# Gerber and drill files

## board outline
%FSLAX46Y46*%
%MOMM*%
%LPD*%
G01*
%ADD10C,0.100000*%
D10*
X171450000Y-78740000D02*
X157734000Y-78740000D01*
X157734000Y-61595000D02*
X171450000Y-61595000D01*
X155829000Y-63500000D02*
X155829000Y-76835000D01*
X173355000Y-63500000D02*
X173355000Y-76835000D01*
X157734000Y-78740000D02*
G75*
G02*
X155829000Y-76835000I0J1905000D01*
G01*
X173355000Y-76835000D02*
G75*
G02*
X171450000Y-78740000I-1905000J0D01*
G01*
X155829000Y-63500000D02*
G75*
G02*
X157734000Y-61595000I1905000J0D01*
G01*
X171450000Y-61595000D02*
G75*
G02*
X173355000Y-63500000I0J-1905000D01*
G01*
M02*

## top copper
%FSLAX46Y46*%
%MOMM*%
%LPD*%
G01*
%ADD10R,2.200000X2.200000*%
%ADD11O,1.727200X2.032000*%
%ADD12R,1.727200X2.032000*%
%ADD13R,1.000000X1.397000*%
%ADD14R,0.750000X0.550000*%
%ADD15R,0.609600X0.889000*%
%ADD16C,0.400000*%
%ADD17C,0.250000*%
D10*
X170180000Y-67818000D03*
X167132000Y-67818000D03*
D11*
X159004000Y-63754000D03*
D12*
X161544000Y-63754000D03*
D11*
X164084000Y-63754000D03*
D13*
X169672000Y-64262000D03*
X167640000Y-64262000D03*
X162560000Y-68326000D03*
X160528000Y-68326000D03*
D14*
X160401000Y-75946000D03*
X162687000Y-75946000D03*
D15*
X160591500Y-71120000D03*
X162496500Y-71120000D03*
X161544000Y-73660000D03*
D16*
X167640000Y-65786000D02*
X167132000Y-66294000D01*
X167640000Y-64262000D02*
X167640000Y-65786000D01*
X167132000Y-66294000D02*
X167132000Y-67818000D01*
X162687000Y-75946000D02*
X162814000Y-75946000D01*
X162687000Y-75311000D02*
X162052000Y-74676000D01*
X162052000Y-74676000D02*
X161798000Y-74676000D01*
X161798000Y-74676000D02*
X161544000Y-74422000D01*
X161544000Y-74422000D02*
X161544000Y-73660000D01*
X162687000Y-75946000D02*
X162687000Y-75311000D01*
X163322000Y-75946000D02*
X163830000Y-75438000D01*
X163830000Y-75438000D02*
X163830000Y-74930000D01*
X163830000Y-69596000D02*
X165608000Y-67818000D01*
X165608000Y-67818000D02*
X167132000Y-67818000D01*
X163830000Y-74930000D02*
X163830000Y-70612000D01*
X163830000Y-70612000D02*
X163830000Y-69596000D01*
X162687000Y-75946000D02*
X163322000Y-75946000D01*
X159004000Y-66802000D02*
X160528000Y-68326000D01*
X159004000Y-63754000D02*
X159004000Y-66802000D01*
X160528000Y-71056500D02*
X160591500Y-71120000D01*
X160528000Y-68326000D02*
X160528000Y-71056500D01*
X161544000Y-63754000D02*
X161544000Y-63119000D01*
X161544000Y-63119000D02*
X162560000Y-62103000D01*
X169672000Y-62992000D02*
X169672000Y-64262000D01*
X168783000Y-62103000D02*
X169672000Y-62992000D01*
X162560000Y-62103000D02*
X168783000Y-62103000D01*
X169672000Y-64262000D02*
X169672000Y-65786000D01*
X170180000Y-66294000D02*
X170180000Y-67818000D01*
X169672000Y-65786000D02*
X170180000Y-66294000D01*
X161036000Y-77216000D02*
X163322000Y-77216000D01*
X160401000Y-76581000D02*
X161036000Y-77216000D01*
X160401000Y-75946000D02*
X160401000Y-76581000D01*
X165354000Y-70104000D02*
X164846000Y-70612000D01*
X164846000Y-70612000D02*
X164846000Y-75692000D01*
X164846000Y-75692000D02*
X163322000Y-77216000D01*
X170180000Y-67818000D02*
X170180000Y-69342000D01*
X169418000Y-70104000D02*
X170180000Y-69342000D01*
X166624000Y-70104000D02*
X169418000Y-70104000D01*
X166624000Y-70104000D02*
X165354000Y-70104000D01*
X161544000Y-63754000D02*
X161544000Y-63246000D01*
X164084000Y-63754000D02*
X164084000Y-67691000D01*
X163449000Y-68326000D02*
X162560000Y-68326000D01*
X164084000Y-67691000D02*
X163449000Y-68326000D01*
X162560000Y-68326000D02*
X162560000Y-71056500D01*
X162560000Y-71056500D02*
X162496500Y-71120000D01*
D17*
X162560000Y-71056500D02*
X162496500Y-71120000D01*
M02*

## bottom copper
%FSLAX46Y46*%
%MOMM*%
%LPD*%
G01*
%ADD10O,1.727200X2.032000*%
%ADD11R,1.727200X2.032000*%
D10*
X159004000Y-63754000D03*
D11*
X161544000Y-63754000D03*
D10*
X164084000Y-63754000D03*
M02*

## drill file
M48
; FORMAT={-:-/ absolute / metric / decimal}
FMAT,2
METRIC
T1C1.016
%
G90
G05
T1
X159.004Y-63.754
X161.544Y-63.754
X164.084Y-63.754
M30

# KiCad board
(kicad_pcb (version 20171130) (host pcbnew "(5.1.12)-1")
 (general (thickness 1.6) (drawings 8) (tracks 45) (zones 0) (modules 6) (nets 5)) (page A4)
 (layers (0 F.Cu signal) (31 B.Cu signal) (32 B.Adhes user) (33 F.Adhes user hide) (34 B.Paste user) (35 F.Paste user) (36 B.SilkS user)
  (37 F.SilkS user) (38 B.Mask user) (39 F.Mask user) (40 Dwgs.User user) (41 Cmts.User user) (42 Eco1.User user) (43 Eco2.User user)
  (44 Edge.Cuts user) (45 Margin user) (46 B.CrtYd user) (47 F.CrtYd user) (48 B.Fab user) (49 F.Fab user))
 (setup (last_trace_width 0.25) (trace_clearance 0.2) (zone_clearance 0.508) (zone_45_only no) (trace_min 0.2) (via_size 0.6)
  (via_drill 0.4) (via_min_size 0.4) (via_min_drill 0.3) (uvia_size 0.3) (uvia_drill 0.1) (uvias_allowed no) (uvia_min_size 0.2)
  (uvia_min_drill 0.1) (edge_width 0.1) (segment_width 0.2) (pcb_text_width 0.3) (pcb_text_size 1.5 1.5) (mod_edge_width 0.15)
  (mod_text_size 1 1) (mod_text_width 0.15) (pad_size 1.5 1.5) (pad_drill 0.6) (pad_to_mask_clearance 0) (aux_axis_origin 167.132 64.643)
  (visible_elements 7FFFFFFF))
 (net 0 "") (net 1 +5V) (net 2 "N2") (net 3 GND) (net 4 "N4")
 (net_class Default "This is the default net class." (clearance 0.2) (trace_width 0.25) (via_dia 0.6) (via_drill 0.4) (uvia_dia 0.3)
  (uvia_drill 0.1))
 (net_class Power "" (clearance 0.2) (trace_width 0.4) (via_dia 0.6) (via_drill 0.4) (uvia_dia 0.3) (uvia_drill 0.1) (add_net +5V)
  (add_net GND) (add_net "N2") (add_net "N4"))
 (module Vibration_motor (layer F.Cu) (at 168.656 67.818 180)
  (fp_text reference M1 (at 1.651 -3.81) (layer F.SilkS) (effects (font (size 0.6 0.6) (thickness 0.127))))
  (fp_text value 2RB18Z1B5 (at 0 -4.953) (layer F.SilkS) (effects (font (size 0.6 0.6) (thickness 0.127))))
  (pad 1 smd rect (at -1.524 0 180) (size 2.2 2.2) (layers F.Cu F.Paste F.Mask) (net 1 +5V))
  (pad 2 smd rect (at 1.524 0 180) (size 2.2 2.2) (layers F.Cu F.Paste F.Mask) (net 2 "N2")))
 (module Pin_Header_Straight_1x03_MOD (layer F.Cu) (at 159.004 63.754 90)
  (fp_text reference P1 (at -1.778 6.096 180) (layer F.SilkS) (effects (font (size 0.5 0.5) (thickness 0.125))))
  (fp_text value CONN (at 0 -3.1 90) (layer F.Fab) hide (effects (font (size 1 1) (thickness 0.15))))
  (pad 1 thru_hole oval (at 0 0 90) (size 2.032 1.7272) (drill 1.016) (layers *.Cu *.Mask F.SilkS) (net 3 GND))
  (pad 2 thru_hole rect (at 0 2.54 90) (size 2.032 1.7272) (drill 1.016) (layers *.Cu *.Mask F.SilkS) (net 1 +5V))
  (pad 3 thru_hole oval (at 0 5.08 90) (size 2.032 1.7272) (drill 1.016) (layers *.Cu *.Mask F.SilkS) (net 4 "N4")))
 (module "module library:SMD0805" (layer F.Cu) (at 168.656 64.262 180)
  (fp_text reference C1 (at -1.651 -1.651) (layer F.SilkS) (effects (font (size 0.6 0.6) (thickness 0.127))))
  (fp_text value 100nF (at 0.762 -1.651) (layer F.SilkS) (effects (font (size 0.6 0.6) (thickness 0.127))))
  (pad 1 smd rect (at -1.016 0 180) (size 1 1.397) (layers F.Cu F.Paste F.Mask) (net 1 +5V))
  (pad 2 smd rect (at 1.016 0 180) (size 1 1.397) (layers F.Cu F.Paste F.Mask) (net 2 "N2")))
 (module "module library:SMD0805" (layer F.Cu) (at 161.544 68.326 180)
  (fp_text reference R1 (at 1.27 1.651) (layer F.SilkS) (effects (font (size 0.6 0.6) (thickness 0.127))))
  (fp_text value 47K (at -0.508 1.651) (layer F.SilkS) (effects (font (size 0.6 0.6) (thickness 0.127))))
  (pad 1 smd rect (at -1.016 0 180) (size 1 1.397) (layers F.Cu F.Paste F.Mask) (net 4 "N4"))
  (pad 2 smd rect (at 1.016 0 180) (size 1 1.397) (layers F.Cu F.Paste F.Mask) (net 3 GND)))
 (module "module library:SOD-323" (layer F.Cu) (at 161.544 75.946)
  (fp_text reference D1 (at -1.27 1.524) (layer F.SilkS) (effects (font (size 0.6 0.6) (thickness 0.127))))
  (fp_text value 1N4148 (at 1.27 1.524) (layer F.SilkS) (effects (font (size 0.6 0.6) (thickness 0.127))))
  (pad 1 smd rect (at -1.143 0) (size 0.75 0.55) (layers F.Cu F.Paste F.Mask) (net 1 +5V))
  (pad 2 smd rect (at 1.143 0) (size 0.75 0.55) (layers F.Cu F.Paste F.Mask) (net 2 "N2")))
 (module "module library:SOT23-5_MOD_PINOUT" (layer F.Cu) (at 161.544 72.39 180)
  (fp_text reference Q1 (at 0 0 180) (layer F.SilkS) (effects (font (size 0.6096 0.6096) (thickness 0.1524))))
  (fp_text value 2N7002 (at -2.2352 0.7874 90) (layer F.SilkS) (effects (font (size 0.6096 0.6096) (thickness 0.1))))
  (pad 3 smd rect (at 0.9525 1.27 180) (size 0.6096 0.889) (layers F.Cu F.Paste F.Mask) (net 3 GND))
  (pad 2 smd rect (at -0.9525 1.27 180) (size 0.6096 0.889) (layers F.Cu F.Paste F.Mask) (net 4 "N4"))
  (pad 1 smd rect (at 0 -1.27 180) (size 0.6096 0.889) (layers F.Cu F.Paste F.Mask) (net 2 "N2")))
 (gr_line (start 171.45 78.74) (end 157.734 78.74) (angle 90) (layer Edge.Cuts) (width 0.1))
 (gr_line (start 157.734 61.595) (end 171.45 61.595) (angle 90) (layer Edge.Cuts) (width 0.1))
 (gr_line (start 155.829 63.5) (end 155.829 76.835) (angle 90) (layer Edge.Cuts) (width 0.1))
 (gr_line (start 173.355 63.5) (end 173.355 76.835) (angle 90) (layer Edge.Cuts) (width 0.1))
 (gr_arc (start 157.734 76.835) (end 157.734 78.74) (angle 90) (layer Edge.Cuts) (width 0.1))
 (gr_arc (start 171.45 76.835) (end 173.355 76.835) (angle 90) (layer Edge.Cuts) (width 0.1))
 (gr_arc (start 157.734 63.5) (end 155.829 63.5) (angle 90) (layer Edge.Cuts) (width 0.1))
 (gr_arc (start 171.45 63.5) (end 171.45 61.595) (angle 90) (layer Edge.Cuts) (width 0.1))
 (segment (start 167.64 65.786) (end 167.132 66.294) (width 0.4) (layer F.Cu) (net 2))
 (segment (start 167.64 64.262) (end 167.64 65.786) (width 0.4) (layer F.Cu) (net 2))
 (segment (start 167.132 66.294) (end 167.132 67.818) (width 0.4) (layer F.Cu) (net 2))
 (segment (start 162.687 75.946) (end 162.814 75.946) (width 0.4) (layer F.Cu) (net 2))
 (segment (start 162.687 75.311) (end 162.052 74.676) (width 0.4) (layer F.Cu) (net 2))
 (segment (start 162.052 74.676) (end 161.798 74.676) (width 0.4) (layer F.Cu) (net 2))
 (segment (start 161.798 74.676) (end 161.544 74.422) (width 0.4) (layer F.Cu) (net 2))
 (segment (start 161.544 74.422) (end 161.544 73.66) (width 0.4) (layer F.Cu) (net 2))
 (segment (start 162.687 75.946) (end 162.687 75.311) (width 0.4) (layer F.Cu) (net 2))
 (segment (start 163.322 75.946) (end 163.83 75.438) (width 0.4) (layer F.Cu) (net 2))
 (segment (start 163.83 75.438) (end 163.83 74.93) (width 0.4) (layer F.Cu) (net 2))
 (segment (start 163.83 69.596) (end 165.608 67.818) (width 0.4) (layer F.Cu) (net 2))
 (segment (start 165.608 67.818) (end 167.132 67.818) (width 0.4) (layer F.Cu) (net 2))
 (segment (start 163.83 74.93) (end 163.83 70.612) (width 0.4) (layer F.Cu) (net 2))
 (segment (start 163.83 70.612) (end 163.83 69.596) (width 0.4) (layer F.Cu) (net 2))
 (segment (start 162.687 75.946) (end 163.322 75.946) (width 0.4) (layer F.Cu) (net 2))
 (segment (start 159.004 66.802) (end 160.528 68.326) (width 0.4) (layer F.Cu) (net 3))
 (segment (start 159.004 63.754) (end 159.004 66.802) (width 0.4) (layer F.Cu) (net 3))
 (segment (start 160.528 71.0565) (end 160.5915 71.12) (width 0.4) (layer F.Cu) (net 3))
 (segment (start 160.528 68.326) (end 160.528 71.0565) (width 0.4) (layer F.Cu) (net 3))
 (segment (start 161.544 63.754) (end 161.544 63.119) (width 0.4) (layer F.Cu) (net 1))
 (segment (start 161.544 63.119) (end 162.56 62.103) (width 0.4) (layer F.Cu) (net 1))
 (segment (start 169.672 62.992) (end 169.672 64.262) (width 0.4) (layer F.Cu) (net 1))
 (segment (start 168.783 62.103) (end 169.672 62.992) (width 0.4) (layer F.Cu) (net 1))
 (segment (start 162.56 62.103) (end 168.783 62.103) (width 0.4) (layer F.Cu) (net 1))
 (segment (start 169.672 64.262) (end 169.672 65.786) (width 0.4) (layer F.Cu) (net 1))
 (segment (start 170.18 66.294) (end 170.18 67.818) (width 0.4) (layer F.Cu) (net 1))
 (segment (start 169.672 65.786) (end 170.18 66.294) (width 0.4) (layer F.Cu) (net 1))
 (segment (start 161.036 77.216) (end 163.322 77.216) (width 0.4) (layer F.Cu) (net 1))
 (segment (start 160.401 76.581) (end 161.036 77.216) (width 0.4) (layer F.Cu) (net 1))
 (segment (start 160.401 75.946) (end 160.401 76.581) (width 0.4) (layer F.Cu) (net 1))
 (segment (start 165.354 70.104) (end 164.846 70.612) (width 0.4) (layer F.Cu) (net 1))
 (segment (start 164.846 70.612) (end 164.846 75.692) (width 0.4) (layer F.Cu) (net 1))
 (segment (start 164.846 75.692) (end 163.322 77.216) (width 0.4) (layer F.Cu) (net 1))
 (segment (start 170.18 67.818) (end 170.18 69.342) (width 0.4) (layer F.Cu) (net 1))
 (segment (start 169.418 70.104) (end 170.18 69.342) (width 0.4) (layer F.Cu) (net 1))
 (segment (start 166.624 70.104) (end 169.418 70.104) (width 0.4) (layer F.Cu) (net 1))
 (segment (start 166.624 70.104) (end 165.354 70.104) (width 0.4) (layer F.Cu) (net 1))
 (segment (start 161.544 63.754) (end 161.544 63.246) (width 0.4) (layer F.Cu) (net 1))
 (segment (start 164.084 63.754) (end 164.084 67.691) (width 0.4) (layer F.Cu) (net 4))
 (segment (start 163.449 68.326) (end 162.56 68.326) (width 0.4) (layer F.Cu) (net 4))
 (segment (start 164.084 67.691) (end 163.449 68.326) (width 0.4) (layer F.Cu) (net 4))
 (segment (start 162.56 68.326) (end 162.56 71.0565) (width 0.4) (layer F.Cu) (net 4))
 (segment (start 162.56 71.0565) (end 162.4965 71.12) (width 0.4) (layer F.Cu) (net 4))
 (segment (start 162.56 71.0565) (end 162.4965 71.12) (width 0.25) (layer F.Cu) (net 4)))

